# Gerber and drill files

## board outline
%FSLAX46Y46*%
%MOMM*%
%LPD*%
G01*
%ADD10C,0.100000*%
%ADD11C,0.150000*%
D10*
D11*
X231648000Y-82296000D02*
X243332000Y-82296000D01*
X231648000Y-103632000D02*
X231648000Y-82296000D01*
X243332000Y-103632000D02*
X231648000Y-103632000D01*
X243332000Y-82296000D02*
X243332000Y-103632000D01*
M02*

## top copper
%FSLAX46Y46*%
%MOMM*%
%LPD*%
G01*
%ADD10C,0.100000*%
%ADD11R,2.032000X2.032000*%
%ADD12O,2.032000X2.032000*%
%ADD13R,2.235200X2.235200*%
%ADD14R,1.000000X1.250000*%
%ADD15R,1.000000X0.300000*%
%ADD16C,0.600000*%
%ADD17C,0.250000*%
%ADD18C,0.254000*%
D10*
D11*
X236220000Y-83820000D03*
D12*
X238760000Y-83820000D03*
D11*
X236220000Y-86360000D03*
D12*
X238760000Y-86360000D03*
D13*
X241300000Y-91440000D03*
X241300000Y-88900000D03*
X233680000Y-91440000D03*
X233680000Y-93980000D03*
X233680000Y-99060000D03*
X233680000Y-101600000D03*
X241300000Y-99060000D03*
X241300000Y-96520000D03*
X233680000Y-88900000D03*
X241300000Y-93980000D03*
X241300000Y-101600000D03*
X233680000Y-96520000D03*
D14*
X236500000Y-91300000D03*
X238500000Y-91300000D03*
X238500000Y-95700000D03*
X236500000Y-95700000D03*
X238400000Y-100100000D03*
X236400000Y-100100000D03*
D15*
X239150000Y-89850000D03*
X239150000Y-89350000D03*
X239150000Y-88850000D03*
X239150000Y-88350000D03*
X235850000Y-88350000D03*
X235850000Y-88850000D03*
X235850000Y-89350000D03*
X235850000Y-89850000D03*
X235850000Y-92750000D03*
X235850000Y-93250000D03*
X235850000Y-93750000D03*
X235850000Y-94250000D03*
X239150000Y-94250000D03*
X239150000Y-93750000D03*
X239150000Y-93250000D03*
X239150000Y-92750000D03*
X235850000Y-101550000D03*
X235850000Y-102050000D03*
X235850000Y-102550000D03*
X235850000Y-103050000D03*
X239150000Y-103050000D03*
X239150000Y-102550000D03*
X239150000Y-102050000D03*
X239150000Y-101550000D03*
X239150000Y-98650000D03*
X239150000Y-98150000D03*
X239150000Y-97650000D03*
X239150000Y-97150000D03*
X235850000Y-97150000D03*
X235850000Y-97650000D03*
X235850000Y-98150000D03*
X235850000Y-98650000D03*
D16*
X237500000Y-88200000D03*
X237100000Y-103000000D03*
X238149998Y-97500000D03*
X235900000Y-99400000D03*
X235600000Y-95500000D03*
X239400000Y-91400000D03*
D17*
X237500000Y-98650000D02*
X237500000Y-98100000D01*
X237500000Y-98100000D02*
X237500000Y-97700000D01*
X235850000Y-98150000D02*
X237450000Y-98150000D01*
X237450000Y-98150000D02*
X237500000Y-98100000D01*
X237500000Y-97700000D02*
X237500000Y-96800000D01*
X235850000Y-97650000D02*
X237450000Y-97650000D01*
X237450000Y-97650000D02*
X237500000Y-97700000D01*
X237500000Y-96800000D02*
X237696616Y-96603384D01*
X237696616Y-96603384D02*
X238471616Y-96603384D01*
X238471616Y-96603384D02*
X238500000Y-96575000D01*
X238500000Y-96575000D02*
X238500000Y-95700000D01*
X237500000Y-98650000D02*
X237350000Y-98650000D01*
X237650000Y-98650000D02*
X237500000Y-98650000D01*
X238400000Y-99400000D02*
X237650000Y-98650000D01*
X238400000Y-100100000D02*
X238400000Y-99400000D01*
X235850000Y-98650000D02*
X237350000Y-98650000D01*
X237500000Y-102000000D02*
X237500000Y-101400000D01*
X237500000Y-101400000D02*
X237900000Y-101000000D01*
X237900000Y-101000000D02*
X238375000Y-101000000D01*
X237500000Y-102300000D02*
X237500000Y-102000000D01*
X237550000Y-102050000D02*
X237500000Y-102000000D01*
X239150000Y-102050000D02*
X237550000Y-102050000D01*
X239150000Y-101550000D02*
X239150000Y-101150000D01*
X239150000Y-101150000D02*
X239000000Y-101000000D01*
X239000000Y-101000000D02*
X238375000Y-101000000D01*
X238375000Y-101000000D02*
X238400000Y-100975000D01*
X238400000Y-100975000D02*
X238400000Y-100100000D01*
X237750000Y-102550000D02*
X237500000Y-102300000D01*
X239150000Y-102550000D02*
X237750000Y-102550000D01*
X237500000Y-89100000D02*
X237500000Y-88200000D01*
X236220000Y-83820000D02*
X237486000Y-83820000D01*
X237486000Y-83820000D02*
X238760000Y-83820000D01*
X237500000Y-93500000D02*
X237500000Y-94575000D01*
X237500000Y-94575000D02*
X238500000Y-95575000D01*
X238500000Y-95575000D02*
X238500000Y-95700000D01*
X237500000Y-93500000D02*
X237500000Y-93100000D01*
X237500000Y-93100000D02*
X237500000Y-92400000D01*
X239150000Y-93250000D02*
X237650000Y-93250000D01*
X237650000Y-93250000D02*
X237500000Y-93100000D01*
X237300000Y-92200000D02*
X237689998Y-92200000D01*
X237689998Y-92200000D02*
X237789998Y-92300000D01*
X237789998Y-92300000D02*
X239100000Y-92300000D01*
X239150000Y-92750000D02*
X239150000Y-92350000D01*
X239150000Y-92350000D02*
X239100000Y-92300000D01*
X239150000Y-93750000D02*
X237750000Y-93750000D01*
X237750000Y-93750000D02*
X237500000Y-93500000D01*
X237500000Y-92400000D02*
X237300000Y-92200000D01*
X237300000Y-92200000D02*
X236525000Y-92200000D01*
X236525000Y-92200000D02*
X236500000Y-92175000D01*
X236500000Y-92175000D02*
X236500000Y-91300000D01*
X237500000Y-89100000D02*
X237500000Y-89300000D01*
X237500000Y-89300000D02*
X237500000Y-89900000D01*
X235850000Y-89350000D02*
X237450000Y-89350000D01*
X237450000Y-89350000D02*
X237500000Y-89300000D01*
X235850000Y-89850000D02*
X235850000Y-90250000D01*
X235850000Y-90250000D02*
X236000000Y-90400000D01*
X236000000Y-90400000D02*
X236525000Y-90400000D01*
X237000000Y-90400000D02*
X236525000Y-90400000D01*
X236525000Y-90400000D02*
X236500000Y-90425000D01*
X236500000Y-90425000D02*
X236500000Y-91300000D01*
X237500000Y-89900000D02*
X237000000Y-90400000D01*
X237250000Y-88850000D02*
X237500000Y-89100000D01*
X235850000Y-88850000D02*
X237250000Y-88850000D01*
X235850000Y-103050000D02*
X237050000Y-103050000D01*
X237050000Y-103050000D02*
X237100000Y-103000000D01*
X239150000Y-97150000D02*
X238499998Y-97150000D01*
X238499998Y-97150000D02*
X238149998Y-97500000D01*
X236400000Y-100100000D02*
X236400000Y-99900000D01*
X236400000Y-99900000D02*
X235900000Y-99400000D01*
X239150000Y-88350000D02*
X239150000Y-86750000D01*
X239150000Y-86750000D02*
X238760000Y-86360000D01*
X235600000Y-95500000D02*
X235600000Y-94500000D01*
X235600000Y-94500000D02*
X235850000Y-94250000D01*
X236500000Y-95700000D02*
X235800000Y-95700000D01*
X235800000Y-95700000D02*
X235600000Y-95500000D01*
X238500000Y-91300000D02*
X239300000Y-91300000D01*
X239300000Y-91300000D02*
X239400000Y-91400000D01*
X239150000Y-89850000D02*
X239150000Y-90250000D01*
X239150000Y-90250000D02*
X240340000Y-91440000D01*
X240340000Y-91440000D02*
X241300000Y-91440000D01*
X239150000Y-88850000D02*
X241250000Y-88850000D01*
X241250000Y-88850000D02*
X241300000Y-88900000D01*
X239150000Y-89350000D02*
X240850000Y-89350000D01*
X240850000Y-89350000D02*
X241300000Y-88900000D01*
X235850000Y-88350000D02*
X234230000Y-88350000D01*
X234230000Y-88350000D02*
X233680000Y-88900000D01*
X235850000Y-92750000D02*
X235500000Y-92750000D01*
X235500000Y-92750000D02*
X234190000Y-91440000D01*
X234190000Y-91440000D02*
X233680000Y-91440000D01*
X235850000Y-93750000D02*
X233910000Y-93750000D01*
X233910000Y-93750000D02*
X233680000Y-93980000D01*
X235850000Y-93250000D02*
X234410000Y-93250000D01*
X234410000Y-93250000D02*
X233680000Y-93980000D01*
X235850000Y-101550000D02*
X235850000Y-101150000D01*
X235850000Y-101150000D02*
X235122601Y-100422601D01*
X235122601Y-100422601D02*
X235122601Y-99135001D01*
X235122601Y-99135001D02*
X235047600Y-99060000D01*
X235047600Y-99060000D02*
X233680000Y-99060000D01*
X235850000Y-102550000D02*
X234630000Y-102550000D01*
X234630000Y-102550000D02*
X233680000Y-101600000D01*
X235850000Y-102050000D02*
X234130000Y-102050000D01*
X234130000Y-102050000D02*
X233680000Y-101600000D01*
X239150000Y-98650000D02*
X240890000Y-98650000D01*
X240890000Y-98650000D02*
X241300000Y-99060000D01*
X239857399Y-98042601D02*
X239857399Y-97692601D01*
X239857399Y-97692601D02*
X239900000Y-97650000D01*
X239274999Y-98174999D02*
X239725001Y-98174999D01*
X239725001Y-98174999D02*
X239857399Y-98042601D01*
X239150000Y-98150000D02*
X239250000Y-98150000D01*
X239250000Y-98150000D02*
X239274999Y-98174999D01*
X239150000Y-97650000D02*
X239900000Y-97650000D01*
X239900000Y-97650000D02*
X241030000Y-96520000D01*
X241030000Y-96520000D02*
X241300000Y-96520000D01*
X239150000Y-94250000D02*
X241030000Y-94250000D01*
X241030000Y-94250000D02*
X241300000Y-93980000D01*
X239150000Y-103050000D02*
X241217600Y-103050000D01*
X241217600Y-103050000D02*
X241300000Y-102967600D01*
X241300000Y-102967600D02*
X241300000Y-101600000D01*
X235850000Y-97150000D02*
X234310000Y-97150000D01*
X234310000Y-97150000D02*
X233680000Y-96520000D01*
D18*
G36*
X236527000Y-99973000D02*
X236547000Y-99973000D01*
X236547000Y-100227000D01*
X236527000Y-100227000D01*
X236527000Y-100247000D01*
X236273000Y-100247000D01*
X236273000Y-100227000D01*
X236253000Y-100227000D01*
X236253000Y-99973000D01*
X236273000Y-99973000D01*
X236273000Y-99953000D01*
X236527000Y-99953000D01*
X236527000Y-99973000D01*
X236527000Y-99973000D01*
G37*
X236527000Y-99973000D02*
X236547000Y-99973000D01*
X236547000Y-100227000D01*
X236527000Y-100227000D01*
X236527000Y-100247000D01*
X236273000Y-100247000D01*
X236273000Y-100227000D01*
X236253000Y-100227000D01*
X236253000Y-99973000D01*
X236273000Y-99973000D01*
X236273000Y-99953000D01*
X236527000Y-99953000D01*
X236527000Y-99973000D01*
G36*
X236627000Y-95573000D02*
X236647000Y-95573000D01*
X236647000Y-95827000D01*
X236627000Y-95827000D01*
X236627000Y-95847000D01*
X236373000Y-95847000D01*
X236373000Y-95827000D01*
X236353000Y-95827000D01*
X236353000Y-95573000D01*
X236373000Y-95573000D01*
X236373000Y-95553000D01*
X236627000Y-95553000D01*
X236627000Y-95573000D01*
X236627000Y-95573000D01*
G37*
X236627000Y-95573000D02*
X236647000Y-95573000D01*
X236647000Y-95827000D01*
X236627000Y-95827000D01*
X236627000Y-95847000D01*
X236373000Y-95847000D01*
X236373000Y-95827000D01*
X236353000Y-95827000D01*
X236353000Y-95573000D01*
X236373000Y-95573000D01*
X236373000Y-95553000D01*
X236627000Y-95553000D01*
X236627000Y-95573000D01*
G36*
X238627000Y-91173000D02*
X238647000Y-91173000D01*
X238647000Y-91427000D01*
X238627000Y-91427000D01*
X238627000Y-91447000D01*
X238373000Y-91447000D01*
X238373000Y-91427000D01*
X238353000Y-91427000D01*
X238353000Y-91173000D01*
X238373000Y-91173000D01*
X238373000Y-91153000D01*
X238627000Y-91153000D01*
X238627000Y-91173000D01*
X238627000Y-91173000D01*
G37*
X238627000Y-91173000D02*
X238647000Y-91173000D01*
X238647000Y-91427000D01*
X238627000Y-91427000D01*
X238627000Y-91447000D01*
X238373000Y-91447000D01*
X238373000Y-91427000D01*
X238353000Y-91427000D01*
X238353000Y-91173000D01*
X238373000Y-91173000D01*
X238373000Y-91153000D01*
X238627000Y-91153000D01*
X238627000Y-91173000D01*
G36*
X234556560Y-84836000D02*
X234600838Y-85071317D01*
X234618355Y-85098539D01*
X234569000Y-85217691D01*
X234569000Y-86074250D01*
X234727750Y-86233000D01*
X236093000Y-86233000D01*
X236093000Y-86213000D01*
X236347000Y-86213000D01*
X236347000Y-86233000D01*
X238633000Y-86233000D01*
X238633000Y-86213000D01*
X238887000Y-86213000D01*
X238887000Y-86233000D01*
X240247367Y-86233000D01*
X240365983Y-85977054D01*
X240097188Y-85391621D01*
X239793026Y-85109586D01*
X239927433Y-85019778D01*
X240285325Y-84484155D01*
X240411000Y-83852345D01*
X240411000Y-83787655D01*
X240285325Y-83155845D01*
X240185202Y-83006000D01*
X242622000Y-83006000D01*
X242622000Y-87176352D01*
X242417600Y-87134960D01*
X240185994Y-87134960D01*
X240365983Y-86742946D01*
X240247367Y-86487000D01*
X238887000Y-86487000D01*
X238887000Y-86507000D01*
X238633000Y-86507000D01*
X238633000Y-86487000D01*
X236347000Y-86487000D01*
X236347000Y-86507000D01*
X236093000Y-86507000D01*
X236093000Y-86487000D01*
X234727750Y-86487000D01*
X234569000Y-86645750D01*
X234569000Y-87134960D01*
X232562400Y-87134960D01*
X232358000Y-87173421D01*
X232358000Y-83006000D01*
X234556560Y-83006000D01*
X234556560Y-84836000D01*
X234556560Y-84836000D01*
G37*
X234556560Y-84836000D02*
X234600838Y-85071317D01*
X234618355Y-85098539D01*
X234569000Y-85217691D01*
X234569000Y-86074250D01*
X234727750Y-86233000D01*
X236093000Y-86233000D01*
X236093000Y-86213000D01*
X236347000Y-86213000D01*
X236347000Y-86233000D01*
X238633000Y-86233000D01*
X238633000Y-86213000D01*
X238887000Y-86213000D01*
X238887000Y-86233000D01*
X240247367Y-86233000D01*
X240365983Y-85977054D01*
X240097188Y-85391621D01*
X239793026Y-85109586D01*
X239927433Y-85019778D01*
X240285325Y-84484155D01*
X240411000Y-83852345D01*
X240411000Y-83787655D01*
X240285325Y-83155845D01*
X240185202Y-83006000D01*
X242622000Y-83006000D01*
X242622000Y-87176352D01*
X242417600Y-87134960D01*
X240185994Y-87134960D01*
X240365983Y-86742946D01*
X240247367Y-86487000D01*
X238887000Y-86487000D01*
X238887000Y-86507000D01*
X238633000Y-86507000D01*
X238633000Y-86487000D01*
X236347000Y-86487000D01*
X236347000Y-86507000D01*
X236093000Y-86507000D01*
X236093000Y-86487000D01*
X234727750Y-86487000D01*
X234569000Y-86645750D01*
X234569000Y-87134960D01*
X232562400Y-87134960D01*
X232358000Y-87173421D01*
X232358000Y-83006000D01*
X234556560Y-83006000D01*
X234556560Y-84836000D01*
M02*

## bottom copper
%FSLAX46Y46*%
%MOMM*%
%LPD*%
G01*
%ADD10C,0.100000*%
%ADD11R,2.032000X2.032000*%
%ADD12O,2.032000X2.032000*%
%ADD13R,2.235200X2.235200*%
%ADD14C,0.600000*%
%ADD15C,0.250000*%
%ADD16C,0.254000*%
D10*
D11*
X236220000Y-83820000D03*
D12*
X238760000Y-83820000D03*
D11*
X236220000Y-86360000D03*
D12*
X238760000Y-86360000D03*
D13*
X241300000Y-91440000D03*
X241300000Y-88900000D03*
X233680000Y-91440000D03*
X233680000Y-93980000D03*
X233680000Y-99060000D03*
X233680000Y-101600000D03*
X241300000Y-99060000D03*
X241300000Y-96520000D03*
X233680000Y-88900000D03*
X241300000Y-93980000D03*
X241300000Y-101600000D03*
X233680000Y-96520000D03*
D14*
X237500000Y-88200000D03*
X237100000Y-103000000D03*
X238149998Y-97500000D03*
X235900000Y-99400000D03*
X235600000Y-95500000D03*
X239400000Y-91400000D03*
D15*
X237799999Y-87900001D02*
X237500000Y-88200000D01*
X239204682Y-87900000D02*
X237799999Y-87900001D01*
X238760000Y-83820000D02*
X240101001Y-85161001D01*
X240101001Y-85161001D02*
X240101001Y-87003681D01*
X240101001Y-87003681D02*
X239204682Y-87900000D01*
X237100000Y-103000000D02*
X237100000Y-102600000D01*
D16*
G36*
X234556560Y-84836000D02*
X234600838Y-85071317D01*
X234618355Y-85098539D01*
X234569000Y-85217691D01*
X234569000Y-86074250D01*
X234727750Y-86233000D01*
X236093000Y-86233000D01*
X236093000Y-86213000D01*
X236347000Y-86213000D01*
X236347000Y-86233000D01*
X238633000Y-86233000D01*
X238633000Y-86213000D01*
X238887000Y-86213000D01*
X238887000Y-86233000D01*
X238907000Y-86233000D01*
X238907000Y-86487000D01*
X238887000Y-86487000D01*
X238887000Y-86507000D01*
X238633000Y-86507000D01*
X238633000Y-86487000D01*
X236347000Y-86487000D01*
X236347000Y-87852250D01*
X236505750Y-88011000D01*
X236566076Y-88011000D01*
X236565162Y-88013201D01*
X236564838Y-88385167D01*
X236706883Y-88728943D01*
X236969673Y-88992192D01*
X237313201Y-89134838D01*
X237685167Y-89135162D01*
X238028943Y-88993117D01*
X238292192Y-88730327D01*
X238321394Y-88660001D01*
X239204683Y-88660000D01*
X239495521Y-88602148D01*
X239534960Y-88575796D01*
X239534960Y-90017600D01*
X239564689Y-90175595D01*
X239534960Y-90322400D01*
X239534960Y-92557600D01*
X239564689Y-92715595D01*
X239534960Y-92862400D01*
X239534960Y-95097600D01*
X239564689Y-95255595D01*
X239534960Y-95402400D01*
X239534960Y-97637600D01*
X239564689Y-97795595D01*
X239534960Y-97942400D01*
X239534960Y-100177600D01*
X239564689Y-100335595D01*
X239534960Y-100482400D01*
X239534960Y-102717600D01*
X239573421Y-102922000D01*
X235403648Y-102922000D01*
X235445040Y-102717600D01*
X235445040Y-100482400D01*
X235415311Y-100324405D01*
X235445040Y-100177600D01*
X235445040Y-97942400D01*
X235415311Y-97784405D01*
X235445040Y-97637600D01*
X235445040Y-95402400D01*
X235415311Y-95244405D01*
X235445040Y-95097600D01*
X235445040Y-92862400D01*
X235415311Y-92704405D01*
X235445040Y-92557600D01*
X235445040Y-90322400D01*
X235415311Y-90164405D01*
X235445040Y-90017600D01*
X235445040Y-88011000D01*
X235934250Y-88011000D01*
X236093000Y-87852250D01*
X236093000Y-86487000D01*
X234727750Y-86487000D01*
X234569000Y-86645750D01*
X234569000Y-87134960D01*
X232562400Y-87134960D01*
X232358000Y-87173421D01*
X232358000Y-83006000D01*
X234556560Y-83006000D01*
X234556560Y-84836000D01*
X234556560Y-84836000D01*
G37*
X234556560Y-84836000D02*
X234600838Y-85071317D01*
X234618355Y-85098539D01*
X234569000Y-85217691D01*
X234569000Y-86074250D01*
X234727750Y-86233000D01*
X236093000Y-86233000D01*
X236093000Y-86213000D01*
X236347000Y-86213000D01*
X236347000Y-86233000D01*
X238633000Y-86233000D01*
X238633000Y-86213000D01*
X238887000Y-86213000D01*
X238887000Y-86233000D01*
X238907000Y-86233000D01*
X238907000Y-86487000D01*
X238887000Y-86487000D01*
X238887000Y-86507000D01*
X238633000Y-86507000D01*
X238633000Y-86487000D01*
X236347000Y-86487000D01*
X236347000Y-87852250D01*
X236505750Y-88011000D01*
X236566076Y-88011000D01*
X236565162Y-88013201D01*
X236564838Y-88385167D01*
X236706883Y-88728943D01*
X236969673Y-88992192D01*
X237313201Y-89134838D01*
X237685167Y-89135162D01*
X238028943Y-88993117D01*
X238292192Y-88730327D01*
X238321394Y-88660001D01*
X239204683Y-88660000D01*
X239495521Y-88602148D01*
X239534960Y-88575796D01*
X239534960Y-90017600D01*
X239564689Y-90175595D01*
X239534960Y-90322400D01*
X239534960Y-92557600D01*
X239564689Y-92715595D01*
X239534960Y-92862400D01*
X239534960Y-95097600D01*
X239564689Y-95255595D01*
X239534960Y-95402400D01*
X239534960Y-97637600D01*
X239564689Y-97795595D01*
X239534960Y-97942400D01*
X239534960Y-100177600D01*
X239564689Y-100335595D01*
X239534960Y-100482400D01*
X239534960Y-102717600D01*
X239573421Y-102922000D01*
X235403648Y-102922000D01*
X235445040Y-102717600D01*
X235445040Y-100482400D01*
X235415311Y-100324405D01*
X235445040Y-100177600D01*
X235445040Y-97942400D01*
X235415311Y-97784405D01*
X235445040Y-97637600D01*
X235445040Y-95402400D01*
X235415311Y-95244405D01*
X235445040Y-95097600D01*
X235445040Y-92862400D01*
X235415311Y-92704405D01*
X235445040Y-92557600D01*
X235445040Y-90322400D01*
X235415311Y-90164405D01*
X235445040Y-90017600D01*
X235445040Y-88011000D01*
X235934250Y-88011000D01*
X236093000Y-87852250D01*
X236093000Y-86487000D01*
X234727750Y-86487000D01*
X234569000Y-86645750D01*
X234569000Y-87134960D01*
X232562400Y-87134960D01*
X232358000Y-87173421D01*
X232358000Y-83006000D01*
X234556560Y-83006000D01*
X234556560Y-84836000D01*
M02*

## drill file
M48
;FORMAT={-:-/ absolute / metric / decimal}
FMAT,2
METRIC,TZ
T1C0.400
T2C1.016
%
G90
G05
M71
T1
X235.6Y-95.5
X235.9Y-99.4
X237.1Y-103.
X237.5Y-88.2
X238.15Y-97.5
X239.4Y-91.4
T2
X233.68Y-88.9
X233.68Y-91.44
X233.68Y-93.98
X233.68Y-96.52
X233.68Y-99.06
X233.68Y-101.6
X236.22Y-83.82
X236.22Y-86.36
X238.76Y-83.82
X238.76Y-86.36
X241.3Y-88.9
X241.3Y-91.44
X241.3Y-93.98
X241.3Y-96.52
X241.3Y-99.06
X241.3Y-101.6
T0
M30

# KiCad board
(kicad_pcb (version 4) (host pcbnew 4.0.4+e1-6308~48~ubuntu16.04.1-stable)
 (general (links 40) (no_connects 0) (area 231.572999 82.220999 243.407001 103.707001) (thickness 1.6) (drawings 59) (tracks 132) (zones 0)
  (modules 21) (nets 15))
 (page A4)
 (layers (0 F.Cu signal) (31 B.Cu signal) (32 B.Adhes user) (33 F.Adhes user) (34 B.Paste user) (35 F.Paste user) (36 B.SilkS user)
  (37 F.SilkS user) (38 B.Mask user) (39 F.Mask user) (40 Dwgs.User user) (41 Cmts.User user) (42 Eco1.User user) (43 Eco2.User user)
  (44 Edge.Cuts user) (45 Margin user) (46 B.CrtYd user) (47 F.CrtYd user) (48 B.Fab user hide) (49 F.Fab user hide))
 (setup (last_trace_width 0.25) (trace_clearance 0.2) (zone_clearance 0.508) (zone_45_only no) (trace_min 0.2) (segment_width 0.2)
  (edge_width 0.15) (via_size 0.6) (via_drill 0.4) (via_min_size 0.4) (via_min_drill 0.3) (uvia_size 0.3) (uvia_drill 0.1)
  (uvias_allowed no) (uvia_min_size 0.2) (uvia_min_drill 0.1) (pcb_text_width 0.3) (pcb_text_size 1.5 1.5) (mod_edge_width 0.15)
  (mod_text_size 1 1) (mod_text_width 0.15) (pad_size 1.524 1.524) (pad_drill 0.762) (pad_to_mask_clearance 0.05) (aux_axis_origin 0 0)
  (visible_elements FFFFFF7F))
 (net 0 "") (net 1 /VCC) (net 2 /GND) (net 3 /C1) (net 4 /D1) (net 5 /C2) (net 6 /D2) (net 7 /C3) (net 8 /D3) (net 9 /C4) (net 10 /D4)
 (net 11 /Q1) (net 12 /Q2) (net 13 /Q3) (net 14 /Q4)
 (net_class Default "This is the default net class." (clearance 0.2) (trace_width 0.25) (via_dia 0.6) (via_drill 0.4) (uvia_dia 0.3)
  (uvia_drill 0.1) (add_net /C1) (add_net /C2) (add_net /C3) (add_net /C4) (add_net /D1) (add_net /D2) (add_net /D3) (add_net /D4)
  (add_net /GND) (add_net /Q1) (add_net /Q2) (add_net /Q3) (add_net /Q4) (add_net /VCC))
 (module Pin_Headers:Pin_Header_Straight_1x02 (layer F.Cu) (at 236.22 83.82 90)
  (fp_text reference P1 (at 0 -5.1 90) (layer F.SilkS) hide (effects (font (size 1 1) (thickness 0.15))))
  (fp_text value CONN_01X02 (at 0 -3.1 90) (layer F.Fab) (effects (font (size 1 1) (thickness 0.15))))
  (pad 1 thru_hole rect (at 0 0 90) (size 2.032 2.032) (drill 1.016) (layers *.Cu *.Mask F.SilkS) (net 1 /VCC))
  (pad 2 thru_hole oval (at 0 2.54 90) (size 2.032 2.032) (drill 1.016) (layers *.Cu *.Mask F.SilkS) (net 1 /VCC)))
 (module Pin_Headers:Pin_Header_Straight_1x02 (layer F.Cu) (at 236.22 86.36 90)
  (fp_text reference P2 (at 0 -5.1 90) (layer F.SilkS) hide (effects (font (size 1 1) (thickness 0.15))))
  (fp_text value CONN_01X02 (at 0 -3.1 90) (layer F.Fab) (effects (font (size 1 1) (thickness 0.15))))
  (pad 1 thru_hole rect (at 0 0 90) (size 2.032 2.032) (drill 1.016) (layers *.Cu *.Mask F.SilkS) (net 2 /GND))
  (pad 2 thru_hole oval (at 0 2.54 90) (size 2.032 2.032) (drill 1.016) (layers *.Cu *.Mask F.SilkS) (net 2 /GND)))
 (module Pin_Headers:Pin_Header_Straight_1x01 (layer F.Cu) (at 241.3 91.44 270)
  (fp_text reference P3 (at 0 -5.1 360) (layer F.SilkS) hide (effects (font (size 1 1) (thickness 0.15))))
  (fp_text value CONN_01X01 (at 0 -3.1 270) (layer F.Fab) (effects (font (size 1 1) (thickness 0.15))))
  (pad 1 thru_hole rect (at 0 0 270) (size 2.2352 2.2352) (drill 1.016) (layers *.Cu *.Mask F.SilkS) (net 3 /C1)))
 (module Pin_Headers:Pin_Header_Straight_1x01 (layer F.Cu) (at 241.3 88.9 270)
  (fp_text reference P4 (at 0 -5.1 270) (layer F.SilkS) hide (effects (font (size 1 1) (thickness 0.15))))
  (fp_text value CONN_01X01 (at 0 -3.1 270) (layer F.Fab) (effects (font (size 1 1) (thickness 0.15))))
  (pad 1 thru_hole rect (at 0 0 270) (size 2.2352 2.2352) (drill 1.016) (layers *.Cu *.Mask F.SilkS) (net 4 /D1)))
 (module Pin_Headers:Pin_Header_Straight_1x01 (layer F.Cu) (at 233.68 91.44 90)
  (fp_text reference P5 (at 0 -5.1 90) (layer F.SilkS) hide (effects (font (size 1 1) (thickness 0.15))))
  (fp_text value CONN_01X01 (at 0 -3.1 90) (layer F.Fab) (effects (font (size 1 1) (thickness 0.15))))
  (pad 1 thru_hole rect (at 0 0 90) (size 2.2352 2.2352) (drill 1.016) (layers *.Cu *.Mask F.SilkS) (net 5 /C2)))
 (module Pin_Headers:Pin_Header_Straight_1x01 (layer F.Cu) (at 233.68 93.98 90)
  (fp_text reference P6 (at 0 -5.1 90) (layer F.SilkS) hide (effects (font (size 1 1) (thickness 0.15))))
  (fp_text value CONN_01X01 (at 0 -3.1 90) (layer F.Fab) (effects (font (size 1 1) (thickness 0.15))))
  (pad 1 thru_hole rect (at 0 0 90) (size 2.2352 2.2352) (drill 1.016) (layers *.Cu *.Mask F.SilkS) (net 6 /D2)))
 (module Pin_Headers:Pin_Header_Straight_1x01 (layer F.Cu) (at 233.68 99.06 90)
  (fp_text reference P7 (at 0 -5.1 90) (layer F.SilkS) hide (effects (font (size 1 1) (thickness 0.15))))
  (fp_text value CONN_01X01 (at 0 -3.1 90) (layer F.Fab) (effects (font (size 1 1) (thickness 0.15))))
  (pad 1 thru_hole rect (at 0 0 90) (size 2.2352 2.2352) (drill 1.016) (layers *.Cu *.Mask F.SilkS) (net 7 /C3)))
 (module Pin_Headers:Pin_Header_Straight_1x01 (layer F.Cu) (at 233.68 101.6 90)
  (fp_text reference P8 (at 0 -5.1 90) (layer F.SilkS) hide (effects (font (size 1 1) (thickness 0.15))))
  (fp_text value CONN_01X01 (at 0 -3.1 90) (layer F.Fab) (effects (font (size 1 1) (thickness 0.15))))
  (pad 1 thru_hole rect (at 0 0 90) (size 2.2352 2.2352) (drill 1.016) (layers *.Cu *.Mask F.SilkS) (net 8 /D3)))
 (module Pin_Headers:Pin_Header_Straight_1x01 (layer F.Cu) (at 241.3 99.06 270)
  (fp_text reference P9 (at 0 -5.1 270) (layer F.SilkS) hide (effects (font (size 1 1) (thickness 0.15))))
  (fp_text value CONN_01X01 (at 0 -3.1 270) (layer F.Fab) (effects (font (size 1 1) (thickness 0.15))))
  (pad 1 thru_hole rect (at 0 0 270) (size 2.2352 2.2352) (drill 1.016) (layers *.Cu *.Mask F.SilkS) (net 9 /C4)))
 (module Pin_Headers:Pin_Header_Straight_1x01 (layer F.Cu) (at 241.3 96.52 270)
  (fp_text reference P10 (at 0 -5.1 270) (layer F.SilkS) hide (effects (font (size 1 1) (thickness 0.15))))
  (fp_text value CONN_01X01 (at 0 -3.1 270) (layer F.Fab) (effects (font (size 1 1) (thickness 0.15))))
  (pad 1 thru_hole rect (at 0 0 270) (size 2.2352 2.2352) (drill 1.016) (layers *.Cu *.Mask F.SilkS) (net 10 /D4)))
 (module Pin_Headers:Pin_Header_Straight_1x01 (layer F.Cu) (at 233.68 88.9 90)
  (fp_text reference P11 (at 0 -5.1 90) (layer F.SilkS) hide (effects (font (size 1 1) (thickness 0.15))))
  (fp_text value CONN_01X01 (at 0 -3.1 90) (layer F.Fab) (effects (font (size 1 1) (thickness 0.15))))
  (pad 1 thru_hole rect (at 0 0 90) (size 2.2352 2.2352) (drill 1.016) (layers *.Cu *.Mask F.SilkS) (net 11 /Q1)))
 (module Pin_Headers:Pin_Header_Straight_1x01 (layer F.Cu) (at 241.3 93.98 270)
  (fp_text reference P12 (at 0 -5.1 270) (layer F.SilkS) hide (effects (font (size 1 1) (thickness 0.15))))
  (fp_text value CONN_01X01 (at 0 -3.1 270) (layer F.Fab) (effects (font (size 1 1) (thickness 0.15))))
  (pad 1 thru_hole rect (at 0 0 270) (size 2.2352 2.2352) (drill 1.016) (layers *.Cu *.Mask F.SilkS) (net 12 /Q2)))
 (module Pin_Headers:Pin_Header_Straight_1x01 (layer F.Cu) (at 241.3 101.6 270)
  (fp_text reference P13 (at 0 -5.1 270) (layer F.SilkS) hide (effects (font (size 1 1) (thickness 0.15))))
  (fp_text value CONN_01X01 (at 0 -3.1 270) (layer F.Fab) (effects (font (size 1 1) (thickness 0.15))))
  (pad 1 thru_hole rect (at 0 0 270) (size 2.2352 2.2352) (drill 1.016) (layers *.Cu *.Mask F.SilkS) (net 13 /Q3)))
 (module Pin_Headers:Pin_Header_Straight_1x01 (layer F.Cu) (at 233.68 96.52 90)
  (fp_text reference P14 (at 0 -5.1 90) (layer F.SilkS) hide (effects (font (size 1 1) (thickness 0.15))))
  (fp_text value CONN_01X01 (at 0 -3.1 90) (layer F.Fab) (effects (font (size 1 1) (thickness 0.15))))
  (pad 1 thru_hole rect (at 0 0 90) (size 2.2352 2.2352) (drill 1.016) (layers *.Cu *.Mask F.SilkS) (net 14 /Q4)))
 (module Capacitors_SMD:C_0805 (layer F.Cu) (at 237.5 91.3)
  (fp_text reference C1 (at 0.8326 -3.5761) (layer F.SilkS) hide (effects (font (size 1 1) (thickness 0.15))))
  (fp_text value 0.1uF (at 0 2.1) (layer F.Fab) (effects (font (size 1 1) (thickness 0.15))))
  (pad 1 smd rect (at -1 0) (size 1 1.25) (layers F.Cu F.Paste F.Mask) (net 1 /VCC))
  (pad 2 smd rect (at 1 0) (size 1 1.25) (layers F.Cu F.Paste F.Mask) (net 2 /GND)))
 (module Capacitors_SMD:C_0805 (layer F.Cu) (at 237.5 95.7 180)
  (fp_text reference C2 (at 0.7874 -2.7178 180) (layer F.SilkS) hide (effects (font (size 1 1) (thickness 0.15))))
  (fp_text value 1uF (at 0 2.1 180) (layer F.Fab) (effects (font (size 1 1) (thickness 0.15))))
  (pad 1 smd rect (at -1 0 180) (size 1 1.25) (layers F.Cu F.Paste F.Mask) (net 1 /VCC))
  (pad 2 smd rect (at 1 0 180) (size 1 1.25) (layers F.Cu F.Paste F.Mask) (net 2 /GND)))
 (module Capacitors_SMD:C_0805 (layer F.Cu) (at 237.4 100.1 180)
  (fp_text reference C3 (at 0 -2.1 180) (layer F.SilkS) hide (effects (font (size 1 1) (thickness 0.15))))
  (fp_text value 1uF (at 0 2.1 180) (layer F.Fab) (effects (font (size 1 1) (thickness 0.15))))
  (pad 1 smd rect (at -1 0 180) (size 1 1.25) (layers F.Cu F.Paste F.Mask) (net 1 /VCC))
  (pad 2 smd rect (at 1 0 180) (size 1 1.25) (layers F.Cu F.Paste F.Mask) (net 2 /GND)))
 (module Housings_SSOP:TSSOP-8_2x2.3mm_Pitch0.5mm (layer F.Cu) (at 237.5 89.1 180)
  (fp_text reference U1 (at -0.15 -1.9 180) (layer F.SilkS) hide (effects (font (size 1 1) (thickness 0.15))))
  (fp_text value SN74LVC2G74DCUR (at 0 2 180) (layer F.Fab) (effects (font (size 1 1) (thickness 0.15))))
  (pad 1 smd rect (at -1.65 -0.75 180) (size 1 0.3) (layers F.Cu F.Paste F.Mask) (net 3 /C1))
  (pad 2 smd rect (at -1.65 -0.25 180) (size 1 0.3) (layers F.Cu F.Paste F.Mask) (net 4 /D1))
  (pad 3 smd rect (at -1.65 0.25 180) (size 1 0.3) (layers F.Cu F.Paste F.Mask) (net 4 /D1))
  (pad 4 smd rect (at -1.65 0.75 180) (size 1 0.3) (layers F.Cu F.Paste F.Mask) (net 2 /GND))
  (pad 5 smd rect (at 1.65 0.75 180) (size 1 0.3) (layers F.Cu F.Paste F.Mask) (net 11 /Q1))
  (pad 6 smd rect (at 1.65 0.25 180) (size 1 0.3) (layers F.Cu F.Paste F.Mask) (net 1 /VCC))
  (pad 7 smd rect (at 1.65 -0.25 180) (size 1 0.3) (layers F.Cu F.Paste F.Mask) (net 1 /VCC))
  (pad 8 smd rect (at 1.65 -0.75 180) (size 1 0.3) (layers F.Cu F.Paste F.Mask) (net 1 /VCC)))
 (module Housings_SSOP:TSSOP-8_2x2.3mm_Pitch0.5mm (layer F.Cu) (at 237.5 93.5)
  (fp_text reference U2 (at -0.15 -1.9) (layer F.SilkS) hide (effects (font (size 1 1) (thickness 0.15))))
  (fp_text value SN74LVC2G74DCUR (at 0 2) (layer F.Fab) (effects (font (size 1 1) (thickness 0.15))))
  (pad 1 smd rect (at -1.65 -0.75) (size 1 0.3) (layers F.Cu F.Paste F.Mask) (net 5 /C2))
  (pad 2 smd rect (at -1.65 -0.25) (size 1 0.3) (layers F.Cu F.Paste F.Mask) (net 6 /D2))
  (pad 3 smd rect (at -1.65 0.25) (size 1 0.3) (layers F.Cu F.Paste F.Mask) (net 6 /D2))
  (pad 4 smd rect (at -1.65 0.75) (size 1 0.3) (layers F.Cu F.Paste F.Mask) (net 2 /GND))
  (pad 5 smd rect (at 1.65 0.75) (size 1 0.3) (layers F.Cu F.Paste F.Mask) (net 12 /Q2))
  (pad 6 smd rect (at 1.65 0.25) (size 1 0.3) (layers F.Cu F.Paste F.Mask) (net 1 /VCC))
  (pad 7 smd rect (at 1.65 -0.25) (size 1 0.3) (layers F.Cu F.Paste F.Mask) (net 1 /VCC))
  (pad 8 smd rect (at 1.65 -0.75) (size 1 0.3) (layers F.Cu F.Paste F.Mask) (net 1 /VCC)))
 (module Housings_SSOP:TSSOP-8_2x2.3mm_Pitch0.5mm (layer F.Cu) (at 237.5 102.3)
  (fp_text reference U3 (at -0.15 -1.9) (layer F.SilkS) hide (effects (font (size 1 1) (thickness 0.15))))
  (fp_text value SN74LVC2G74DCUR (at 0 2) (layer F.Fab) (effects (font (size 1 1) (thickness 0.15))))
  (pad 1 smd rect (at -1.65 -0.75) (size 1 0.3) (layers F.Cu F.Paste F.Mask) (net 7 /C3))
  (pad 2 smd rect (at -1.65 -0.25) (size 1 0.3) (layers F.Cu F.Paste F.Mask) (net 8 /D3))
  (pad 3 smd rect (at -1.65 0.25) (size 1 0.3) (layers F.Cu F.Paste F.Mask) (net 8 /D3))
  (pad 4 smd rect (at -1.65 0.75) (size 1 0.3) (layers F.Cu F.Paste F.Mask) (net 2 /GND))
  (pad 5 smd rect (at 1.65 0.75) (size 1 0.3) (layers F.Cu F.Paste F.Mask) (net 13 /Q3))
  (pad 6 smd rect (at 1.65 0.25) (size 1 0.3) (layers F.Cu F.Paste F.Mask) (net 1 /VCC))
  (pad 7 smd rect (at 1.65 -0.25) (size 1 0.3) (layers F.Cu F.Paste F.Mask) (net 1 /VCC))
  (pad 8 smd rect (at 1.65 -0.75) (size 1 0.3) (layers F.Cu F.Paste F.Mask) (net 1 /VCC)))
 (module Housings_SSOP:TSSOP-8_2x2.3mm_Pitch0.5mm (layer F.Cu) (at 237.5 97.9 180)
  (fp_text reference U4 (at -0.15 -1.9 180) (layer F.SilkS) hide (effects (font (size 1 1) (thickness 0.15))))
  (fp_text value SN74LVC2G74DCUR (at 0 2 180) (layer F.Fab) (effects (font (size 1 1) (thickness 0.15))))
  (pad 1 smd rect (at -1.65 -0.75 180) (size 1 0.3) (layers F.Cu F.Paste F.Mask) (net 9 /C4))
  (pad 2 smd rect (at -1.65 -0.25 180) (size 1 0.3) (layers F.Cu F.Paste F.Mask) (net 10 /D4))
  (pad 3 smd rect (at -1.65 0.25 180) (size 1 0.3) (layers F.Cu F.Paste F.Mask) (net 10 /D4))
  (pad 4 smd rect (at -1.65 0.75 180) (size 1 0.3) (layers F.Cu F.Paste F.Mask) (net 2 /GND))
  (pad 5 smd rect (at 1.65 0.75 180) (size 1 0.3) (layers F.Cu F.Paste F.Mask) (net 14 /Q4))
  (pad 6 smd rect (at 1.65 0.25 180) (size 1 0.3) (layers F.Cu F.Paste F.Mask) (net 1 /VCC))
  (pad 7 smd rect (at 1.65 -0.25 180) (size 1 0.3) (layers F.Cu F.Paste F.Mask) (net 1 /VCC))
  (pad 8 smd rect (at 1.65 -0.75 180) (size 1 0.3) (layers F.Cu F.Paste F.Mask) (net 1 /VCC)))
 (gr_line (start 231.648 82.296) (end 243.332 82.296) (layer Edge.Cuts) (width 0.15))
 (gr_line (start 231.648 103.632) (end 231.648 82.296) (layer Edge.Cuts) (width 0.15))
 (gr_line (start 243.332 103.632) (end 231.648 103.632) (layer Edge.Cuts) (width 0.15))
 (gr_line (start 243.332 82.296) (end 243.332 103.632) (layer Edge.Cuts) (width 0.15))
 (via (at 237.5 88.2) (size 0.6) (drill 0.4) (layers F.Cu B.Cu) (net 1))
 (segment (start 237.799999 87.900001) (end 237.5 88.2) (width 0.25) (layer B.Cu) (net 1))
 (segment (start 239.204682 87.9) (end 237.799999 87.900001) (width 0.25) (layer B.Cu) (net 1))
 (segment (start 237.5 98.65) (end 237.5 98.1) (width 0.25) (layer F.Cu) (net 1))
 (segment (start 237.5 98.1) (end 237.5 97.7) (width 0.25) (layer F.Cu) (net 1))
 (segment (start 235.85 98.15) (end 237.45 98.15) (width 0.25) (layer F.Cu) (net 1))
 (segment (start 237.45 98.15) (end 237.5 98.1) (width 0.25) (layer F.Cu) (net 1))
 (segment (start 237.5 97.7) (end 237.5 96.8) (width 0.25) (layer F.Cu) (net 1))
 (segment (start 235.85 97.65) (end 237.45 97.65) (width 0.25) (layer F.Cu) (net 1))
 (segment (start 237.45 97.65) (end 237.5 97.7) (width 0.25) (layer F.Cu) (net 1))
 (segment (start 237.5 96.8) (end 237.696616 96.603384) (width 0.25) (layer F.Cu) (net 1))
 (segment (start 237.696616 96.603384) (end 238.471616 96.603384) (width 0.25) (layer F.Cu) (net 1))
 (segment (start 238.471616 96.603384) (end 238.5 96.575) (width 0.25) (layer F.Cu) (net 1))
 (segment (start 238.5 96.575) (end 238.5 95.7) (width 0.25) (layer F.Cu) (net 1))
 (segment (start 237.5 98.65) (end 237.35 98.65) (width 0.25) (layer F.Cu) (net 1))
 (segment (start 237.65 98.65) (end 237.5 98.65) (width 0.25) (layer F.Cu) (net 1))
 (segment (start 238.4 99.4) (end 237.65 98.65) (width 0.25) (layer F.Cu) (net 1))
 (segment (start 238.4 100.1) (end 238.4 99.4) (width 0.25) (layer F.Cu) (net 1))
 (segment (start 235.85 98.65) (end 237.35 98.65) (width 0.25) (layer F.Cu) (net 1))
 (segment (start 237.5 102) (end 237.5 101.4) (width 0.25) (layer F.Cu) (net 1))
 (segment (start 237.5 101.4) (end 237.9 101) (width 0.25) (layer F.Cu) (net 1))
 (segment (start 237.9 101) (end 238.375 101) (width 0.25) (layer F.Cu) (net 1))
 (segment (start 237.5 102.3) (end 237.5 102) (width 0.25) (layer F.Cu) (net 1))
 (segment (start 237.55 102.05) (end 237.5 102) (width 0.25) (layer F.Cu) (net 1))
 (segment (start 239.15 102.05) (end 237.55 102.05) (width 0.25) (layer F.Cu) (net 1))
 (segment (start 239.15 101.55) (end 239.15 101.15) (width 0.25) (layer F.Cu) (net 1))
 (segment (start 239.15 101.15) (end 239 101) (width 0.25) (layer F.Cu) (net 1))
 (segment (start 239 101) (end 238.375 101) (width 0.25) (layer F.Cu) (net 1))
 (segment (start 238.375 101) (end 238.4 100.975) (width 0.25) (layer F.Cu) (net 1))
 (segment (start 238.4 100.975) (end 238.4 100.1) (width 0.25) (layer F.Cu) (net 1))
 (segment (start 237.75 102.55) (end 237.5 102.3) (width 0.25) (layer F.Cu) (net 1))
 (segment (start 239.15 102.55) (end 237.75 102.55) (width 0.25) (layer F.Cu) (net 1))
 (segment (start 238.76 83.82) (end 240.101001 85.161001) (width 0.25) (layer B.Cu) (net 1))
 (segment (start 240.101001 85.161001) (end 240.101001 87.003681) (width 0.25) (layer B.Cu) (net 1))
 (segment (start 240.101001 87.003681) (end 239.204682 87.9) (width 0.25) (layer B.Cu) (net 1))
 (segment (start 237.5 89.1) (end 237.5 88.2) (width 0.25) (layer F.Cu) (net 1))
 (segment (start 236.22 83.82) (end 237.486 83.82) (width 0.25) (layer F.Cu) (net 1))
 (segment (start 237.486 83.82) (end 238.76 83.82) (width 0.25) (layer F.Cu) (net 1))
 (segment (start 237.5 93.5) (end 237.5 94.575) (width 0.25) (layer F.Cu) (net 1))
 (segment (start 237.5 94.575) (end 238.5 95.575) (width 0.25) (layer F.Cu) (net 1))
 (segment (start 238.5 95.575) (end 238.5 95.7) (width 0.25) (layer F.Cu) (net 1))
 (segment (start 237.5 93.5) (end 237.5 93.1) (width 0.25) (layer F.Cu) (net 1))
 (segment (start 237.5 93.1) (end 237.5 92.4) (width 0.25) (layer F.Cu) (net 1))
 (segment (start 239.15 93.25) (end 237.65 93.25) (width 0.25) (layer F.Cu) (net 1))
 (segment (start 237.65 93.25) (end 237.5 93.1) (width 0.25) (layer F.Cu) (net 1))
 (segment (start 237.3 92.2) (end 237.689998 92.2) (width 0.25) (layer F.Cu) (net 1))
 (segment (start 237.689998 92.2) (end 237.789998 92.3) (width 0.25) (layer F.Cu) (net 1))
 (segment (start 237.789998 92.3) (end 239.1 92.3) (width 0.25) (layer F.Cu) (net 1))
 (segment (start 239.15 92.75) (end 239.15 92.35) (width 0.25) (layer F.Cu) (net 1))
 (segment (start 239.15 92.35) (end 239.1 92.3) (width 0.25) (layer F.Cu) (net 1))
 (segment (start 239.15 93.75) (end 237.75 93.75) (width 0.25) (layer F.Cu) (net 1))
 (segment (start 237.75 93.75) (end 237.5 93.5) (width 0.25) (layer F.Cu) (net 1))
 (segment (start 237.5 92.4) (end 237.3 92.2) (width 0.25) (layer F.Cu) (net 1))
 (segment (start 237.3 92.2) (end 236.525 92.2) (width 0.25) (layer F.Cu) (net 1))
 (segment (start 236.525 92.2) (end 236.5 92.175) (width 0.25) (layer F.Cu) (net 1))
 (segment (start 236.5 92.175) (end 236.5 91.3) (width 0.25) (layer F.Cu) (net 1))
 (segment (start 237.5 89.1) (end 237.5 89.3) (width 0.25) (layer F.Cu) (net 1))
 (segment (start 237.5 89.3) (end 237.5 89.9) (width 0.25) (layer F.Cu) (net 1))
 (segment (start 235.85 89.35) (end 237.45 89.35) (width 0.25) (layer F.Cu) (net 1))
 (segment (start 237.45 89.35) (end 237.5 89.3) (width 0.25) (layer F.Cu) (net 1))
 (segment (start 235.85 89.85) (end 235.85 90.25) (width 0.25) (layer F.Cu) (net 1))
 (segment (start 235.85 90.25) (end 236 90.4) (width 0.25) (layer F.Cu) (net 1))
 (segment (start 236 90.4) (end 236.525 90.4) (width 0.25) (layer F.Cu) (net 1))
 (segment (start 237 90.4) (end 236.525 90.4) (width 0.25) (layer F.Cu) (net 1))
 (segment (start 236.525 90.4) (end 236.5 90.425) (width 0.25) (layer F.Cu) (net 1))
 (segment (start 236.5 90.425) (end 236.5 91.3) (width 0.25) (layer F.Cu) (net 1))
 (segment (start 237.5 89.9) (end 237 90.4) (width 0.25) (layer F.Cu) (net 1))
 (segment (start 237.25 88.85) (end 237.5 89.1) (width 0.25) (layer F.Cu) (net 1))
 (segment (start 235.85 88.85) (end 237.25 88.85) (width 0.25) (layer F.Cu) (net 1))
 (segment (start 237.1 103) (end 237.1 102.6) (width 0.25) (layer B.Cu) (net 2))
 (segment (start 235.85 103.05) (end 237.05 103.05) (width 0.25) (layer F.Cu) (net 2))
 (segment (start 237.05 103.05) (end 237.1 103) (width 0.25) (layer F.Cu) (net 2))
 (via (at 237.1 103) (size 0.6) (drill 0.4) (layers F.Cu B.Cu) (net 2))
 (segment (start 239.15 97.15) (end 238.499998 97.15) (width 0.25) (layer F.Cu) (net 2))
 (segment (start 238.499998 97.15) (end 238.149998 97.5) (width 0.25) (layer F.Cu) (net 2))
 (via (at 238.149998 97.5) (size 0.6) (drill 0.4) (layers F.Cu B.Cu) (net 2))
 (segment (start 236.4 100.1) (end 236.4 99.9) (width 0.25) (layer F.Cu) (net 2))
 (segment (start 236.4 99.9) (end 235.9 99.4) (width 0.25) (layer F.Cu) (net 2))
 (via (at 235.9 99.4) (size 0.6) (drill 0.4) (layers F.Cu B.Cu) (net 2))
 (segment (start 239.15 88.35) (end 239.15 86.75) (width 0.25) (layer F.Cu) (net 2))
 (segment (start 239.15 86.75) (end 238.76 86.36) (width 0.25) (layer F.Cu) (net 2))
 (segment (start 235.6 95.5) (end 235.6 94.5) (width 0.25) (layer F.Cu) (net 2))
 (segment (start 235.6 94.5) (end 235.85 94.25) (width 0.25) (layer F.Cu) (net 2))
 (segment (start 236.5 95.7) (end 235.8 95.7) (width 0.25) (layer F.Cu) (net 2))
 (segment (start 235.8 95.7) (end 235.6 95.5) (width 0.25) (layer F.Cu) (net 2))
 (via (at 235.6 95.5) (size 0.6) (drill 0.4) (layers F.Cu B.Cu) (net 2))
 (segment (start 238.5 91.3) (end 239.3 91.3) (width 0.25) (layer F.Cu) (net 2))
 (segment (start 239.3 91.3) (end 239.4 91.4) (width 0.25) (layer F.Cu) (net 2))
 (via (at 239.4 91.4) (size 0.6) (drill 0.4) (layers F.Cu B.Cu) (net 2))
 (segment (start 239.15 89.85) (end 239.15 90.25) (width 0.25) (layer F.Cu) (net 3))
 (segment (start 239.15 90.25) (end 240.34 91.44) (width 0.25) (layer F.Cu) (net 3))
 (segment (start 240.34 91.44) (end 241.3 91.44) (width 0.25) (layer F.Cu) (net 3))
 (segment (start 239.15 88.85) (end 241.25 88.85) (width 0.25) (layer F.Cu) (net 4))
 (segment (start 241.25 88.85) (end 241.3 88.9) (width 0.25) (layer F.Cu) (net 4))
 (segment (start 239.15 89.35) (end 240.85 89.35) (width 0.25) (layer F.Cu) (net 4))
 (segment (start 240.85 89.35) (end 241.3 88.9) (width 0.25) (layer F.Cu) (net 4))
 (segment (start 235.85 88.35) (end 234.23 88.35) (width 0.25) (layer F.Cu) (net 11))
 (segment (start 234.23 88.35) (end 233.68 88.9) (width 0.25) (layer F.Cu) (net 11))
 (segment (start 235.85 92.75) (end 235.5 92.75) (width 0.25) (layer F.Cu) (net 5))
 (segment (start 235.5 92.75) (end 234.19 91.44) (width 0.25) (layer F.Cu) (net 5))
 (segment (start 234.19 91.44) (end 233.68 91.44) (width 0.25) (layer F.Cu) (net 5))
 (segment (start 235.85 93.75) (end 233.91 93.75) (width 0.25) (layer F.Cu) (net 6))
 (segment (start 233.91 93.75) (end 233.68 93.98) (width 0.25) (layer F.Cu) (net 6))
 (segment (start 235.85 93.25) (end 234.41 93.25) (width 0.25) (layer F.Cu) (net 6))
 (segment (start 234.41 93.25) (end 233.68 93.98) (width 0.25) (layer F.Cu) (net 6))
 (segment (start 235.85 101.55) (end 235.85 101.15) (width 0.25) (layer F.Cu) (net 7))
 (segment (start 235.85 101.15) (end 235.122601 100.422601) (width 0.25) (layer F.Cu) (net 7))
 (segment (start 235.122601 100.422601) (end 235.122601 99.135001) (width 0.25) (layer F.Cu) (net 7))
 (segment (start 235.122601 99.135001) (end 235.0476 99.06) (width 0.25) (layer F.Cu) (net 7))
 (segment (start 235.0476 99.06) (end 233.68 99.06) (width 0.25) (layer F.Cu) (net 7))
 (segment (start 235.85 102.55) (end 234.63 102.55) (width 0.25) (layer F.Cu) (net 8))
 (segment (start 234.63 102.55) (end 233.68 101.6) (width 0.25) (layer F.Cu) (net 8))
 (segment (start 235.85 102.05) (end 234.13 102.05) (width 0.25) (layer F.Cu) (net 8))
 (segment (start 234.13 102.05) (end 233.68 101.6) (width 0.25) (layer F.Cu) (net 8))
 (segment (start 239.15 98.65) (end 240.89 98.65) (width 0.25) (layer F.Cu) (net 9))
 (segment (start 240.89 98.65) (end 241.3 99.06) (width 0.25) (layer F.Cu) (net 9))
 (segment (start 239.857399 98.042601) (end 239.857399 97.692601) (width 0.25) (layer F.Cu) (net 10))
 (segment (start 239.857399 97.692601) (end 239.9 97.65) (width 0.25) (layer F.Cu) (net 10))
 (segment (start 239.274999 98.174999) (end 239.725001 98.174999) (width 0.25) (layer F.Cu) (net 10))
 (segment (start 239.725001 98.174999) (end 239.857399 98.042601) (width 0.25) (layer F.Cu) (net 10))
 (segment (start 239.15 98.15) (end 239.25 98.15) (width 0.25) (layer F.Cu) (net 10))
 (segment (start 239.25 98.15) (end 239.274999 98.174999) (width 0.25) (layer F.Cu) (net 10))
 (segment (start 239.15 97.65) (end 239.9 97.65) (width 0.25) (layer F.Cu) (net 10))
 (segment (start 239.9 97.65) (end 241.03 96.52) (width 0.25) (layer F.Cu) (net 10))
 (segment (start 241.03 96.52) (end 241.3 96.52) (width 0.25) (layer F.Cu) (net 10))
 (segment (start 239.15 94.25) (end 241.03 94.25) (width 0.25) (layer F.Cu) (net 12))
 (segment (start 241.03 94.25) (end 241.3 93.98) (width 0.25) (layer F.Cu) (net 12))
 (segment (start 239.15 103.05) (end 241.2176 103.05) (width 0.25) (layer F.Cu) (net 13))
 (segment (start 241.2176 103.05) (end 241.3 102.9676) (width 0.25) (layer F.Cu) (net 13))
 (segment (start 241.3 102.9676) (end 241.3 101.6) (width 0.25) (layer F.Cu) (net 13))
 (segment (start 235.85 97.15) (end 234.31 97.15) (width 0.25) (layer F.Cu) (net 14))
 (segment (start 234.31 97.15) (end 233.68 96.52) (width 0.25) (layer F.Cu) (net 14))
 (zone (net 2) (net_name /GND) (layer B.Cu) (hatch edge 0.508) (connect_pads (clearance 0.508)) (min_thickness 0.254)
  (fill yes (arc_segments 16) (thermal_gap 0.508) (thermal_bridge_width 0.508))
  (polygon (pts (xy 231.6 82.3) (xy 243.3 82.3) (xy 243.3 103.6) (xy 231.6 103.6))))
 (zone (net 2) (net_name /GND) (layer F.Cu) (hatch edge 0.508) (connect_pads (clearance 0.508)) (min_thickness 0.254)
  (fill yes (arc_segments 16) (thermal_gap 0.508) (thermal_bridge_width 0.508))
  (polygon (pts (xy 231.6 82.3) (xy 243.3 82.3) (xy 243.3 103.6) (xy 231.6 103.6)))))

